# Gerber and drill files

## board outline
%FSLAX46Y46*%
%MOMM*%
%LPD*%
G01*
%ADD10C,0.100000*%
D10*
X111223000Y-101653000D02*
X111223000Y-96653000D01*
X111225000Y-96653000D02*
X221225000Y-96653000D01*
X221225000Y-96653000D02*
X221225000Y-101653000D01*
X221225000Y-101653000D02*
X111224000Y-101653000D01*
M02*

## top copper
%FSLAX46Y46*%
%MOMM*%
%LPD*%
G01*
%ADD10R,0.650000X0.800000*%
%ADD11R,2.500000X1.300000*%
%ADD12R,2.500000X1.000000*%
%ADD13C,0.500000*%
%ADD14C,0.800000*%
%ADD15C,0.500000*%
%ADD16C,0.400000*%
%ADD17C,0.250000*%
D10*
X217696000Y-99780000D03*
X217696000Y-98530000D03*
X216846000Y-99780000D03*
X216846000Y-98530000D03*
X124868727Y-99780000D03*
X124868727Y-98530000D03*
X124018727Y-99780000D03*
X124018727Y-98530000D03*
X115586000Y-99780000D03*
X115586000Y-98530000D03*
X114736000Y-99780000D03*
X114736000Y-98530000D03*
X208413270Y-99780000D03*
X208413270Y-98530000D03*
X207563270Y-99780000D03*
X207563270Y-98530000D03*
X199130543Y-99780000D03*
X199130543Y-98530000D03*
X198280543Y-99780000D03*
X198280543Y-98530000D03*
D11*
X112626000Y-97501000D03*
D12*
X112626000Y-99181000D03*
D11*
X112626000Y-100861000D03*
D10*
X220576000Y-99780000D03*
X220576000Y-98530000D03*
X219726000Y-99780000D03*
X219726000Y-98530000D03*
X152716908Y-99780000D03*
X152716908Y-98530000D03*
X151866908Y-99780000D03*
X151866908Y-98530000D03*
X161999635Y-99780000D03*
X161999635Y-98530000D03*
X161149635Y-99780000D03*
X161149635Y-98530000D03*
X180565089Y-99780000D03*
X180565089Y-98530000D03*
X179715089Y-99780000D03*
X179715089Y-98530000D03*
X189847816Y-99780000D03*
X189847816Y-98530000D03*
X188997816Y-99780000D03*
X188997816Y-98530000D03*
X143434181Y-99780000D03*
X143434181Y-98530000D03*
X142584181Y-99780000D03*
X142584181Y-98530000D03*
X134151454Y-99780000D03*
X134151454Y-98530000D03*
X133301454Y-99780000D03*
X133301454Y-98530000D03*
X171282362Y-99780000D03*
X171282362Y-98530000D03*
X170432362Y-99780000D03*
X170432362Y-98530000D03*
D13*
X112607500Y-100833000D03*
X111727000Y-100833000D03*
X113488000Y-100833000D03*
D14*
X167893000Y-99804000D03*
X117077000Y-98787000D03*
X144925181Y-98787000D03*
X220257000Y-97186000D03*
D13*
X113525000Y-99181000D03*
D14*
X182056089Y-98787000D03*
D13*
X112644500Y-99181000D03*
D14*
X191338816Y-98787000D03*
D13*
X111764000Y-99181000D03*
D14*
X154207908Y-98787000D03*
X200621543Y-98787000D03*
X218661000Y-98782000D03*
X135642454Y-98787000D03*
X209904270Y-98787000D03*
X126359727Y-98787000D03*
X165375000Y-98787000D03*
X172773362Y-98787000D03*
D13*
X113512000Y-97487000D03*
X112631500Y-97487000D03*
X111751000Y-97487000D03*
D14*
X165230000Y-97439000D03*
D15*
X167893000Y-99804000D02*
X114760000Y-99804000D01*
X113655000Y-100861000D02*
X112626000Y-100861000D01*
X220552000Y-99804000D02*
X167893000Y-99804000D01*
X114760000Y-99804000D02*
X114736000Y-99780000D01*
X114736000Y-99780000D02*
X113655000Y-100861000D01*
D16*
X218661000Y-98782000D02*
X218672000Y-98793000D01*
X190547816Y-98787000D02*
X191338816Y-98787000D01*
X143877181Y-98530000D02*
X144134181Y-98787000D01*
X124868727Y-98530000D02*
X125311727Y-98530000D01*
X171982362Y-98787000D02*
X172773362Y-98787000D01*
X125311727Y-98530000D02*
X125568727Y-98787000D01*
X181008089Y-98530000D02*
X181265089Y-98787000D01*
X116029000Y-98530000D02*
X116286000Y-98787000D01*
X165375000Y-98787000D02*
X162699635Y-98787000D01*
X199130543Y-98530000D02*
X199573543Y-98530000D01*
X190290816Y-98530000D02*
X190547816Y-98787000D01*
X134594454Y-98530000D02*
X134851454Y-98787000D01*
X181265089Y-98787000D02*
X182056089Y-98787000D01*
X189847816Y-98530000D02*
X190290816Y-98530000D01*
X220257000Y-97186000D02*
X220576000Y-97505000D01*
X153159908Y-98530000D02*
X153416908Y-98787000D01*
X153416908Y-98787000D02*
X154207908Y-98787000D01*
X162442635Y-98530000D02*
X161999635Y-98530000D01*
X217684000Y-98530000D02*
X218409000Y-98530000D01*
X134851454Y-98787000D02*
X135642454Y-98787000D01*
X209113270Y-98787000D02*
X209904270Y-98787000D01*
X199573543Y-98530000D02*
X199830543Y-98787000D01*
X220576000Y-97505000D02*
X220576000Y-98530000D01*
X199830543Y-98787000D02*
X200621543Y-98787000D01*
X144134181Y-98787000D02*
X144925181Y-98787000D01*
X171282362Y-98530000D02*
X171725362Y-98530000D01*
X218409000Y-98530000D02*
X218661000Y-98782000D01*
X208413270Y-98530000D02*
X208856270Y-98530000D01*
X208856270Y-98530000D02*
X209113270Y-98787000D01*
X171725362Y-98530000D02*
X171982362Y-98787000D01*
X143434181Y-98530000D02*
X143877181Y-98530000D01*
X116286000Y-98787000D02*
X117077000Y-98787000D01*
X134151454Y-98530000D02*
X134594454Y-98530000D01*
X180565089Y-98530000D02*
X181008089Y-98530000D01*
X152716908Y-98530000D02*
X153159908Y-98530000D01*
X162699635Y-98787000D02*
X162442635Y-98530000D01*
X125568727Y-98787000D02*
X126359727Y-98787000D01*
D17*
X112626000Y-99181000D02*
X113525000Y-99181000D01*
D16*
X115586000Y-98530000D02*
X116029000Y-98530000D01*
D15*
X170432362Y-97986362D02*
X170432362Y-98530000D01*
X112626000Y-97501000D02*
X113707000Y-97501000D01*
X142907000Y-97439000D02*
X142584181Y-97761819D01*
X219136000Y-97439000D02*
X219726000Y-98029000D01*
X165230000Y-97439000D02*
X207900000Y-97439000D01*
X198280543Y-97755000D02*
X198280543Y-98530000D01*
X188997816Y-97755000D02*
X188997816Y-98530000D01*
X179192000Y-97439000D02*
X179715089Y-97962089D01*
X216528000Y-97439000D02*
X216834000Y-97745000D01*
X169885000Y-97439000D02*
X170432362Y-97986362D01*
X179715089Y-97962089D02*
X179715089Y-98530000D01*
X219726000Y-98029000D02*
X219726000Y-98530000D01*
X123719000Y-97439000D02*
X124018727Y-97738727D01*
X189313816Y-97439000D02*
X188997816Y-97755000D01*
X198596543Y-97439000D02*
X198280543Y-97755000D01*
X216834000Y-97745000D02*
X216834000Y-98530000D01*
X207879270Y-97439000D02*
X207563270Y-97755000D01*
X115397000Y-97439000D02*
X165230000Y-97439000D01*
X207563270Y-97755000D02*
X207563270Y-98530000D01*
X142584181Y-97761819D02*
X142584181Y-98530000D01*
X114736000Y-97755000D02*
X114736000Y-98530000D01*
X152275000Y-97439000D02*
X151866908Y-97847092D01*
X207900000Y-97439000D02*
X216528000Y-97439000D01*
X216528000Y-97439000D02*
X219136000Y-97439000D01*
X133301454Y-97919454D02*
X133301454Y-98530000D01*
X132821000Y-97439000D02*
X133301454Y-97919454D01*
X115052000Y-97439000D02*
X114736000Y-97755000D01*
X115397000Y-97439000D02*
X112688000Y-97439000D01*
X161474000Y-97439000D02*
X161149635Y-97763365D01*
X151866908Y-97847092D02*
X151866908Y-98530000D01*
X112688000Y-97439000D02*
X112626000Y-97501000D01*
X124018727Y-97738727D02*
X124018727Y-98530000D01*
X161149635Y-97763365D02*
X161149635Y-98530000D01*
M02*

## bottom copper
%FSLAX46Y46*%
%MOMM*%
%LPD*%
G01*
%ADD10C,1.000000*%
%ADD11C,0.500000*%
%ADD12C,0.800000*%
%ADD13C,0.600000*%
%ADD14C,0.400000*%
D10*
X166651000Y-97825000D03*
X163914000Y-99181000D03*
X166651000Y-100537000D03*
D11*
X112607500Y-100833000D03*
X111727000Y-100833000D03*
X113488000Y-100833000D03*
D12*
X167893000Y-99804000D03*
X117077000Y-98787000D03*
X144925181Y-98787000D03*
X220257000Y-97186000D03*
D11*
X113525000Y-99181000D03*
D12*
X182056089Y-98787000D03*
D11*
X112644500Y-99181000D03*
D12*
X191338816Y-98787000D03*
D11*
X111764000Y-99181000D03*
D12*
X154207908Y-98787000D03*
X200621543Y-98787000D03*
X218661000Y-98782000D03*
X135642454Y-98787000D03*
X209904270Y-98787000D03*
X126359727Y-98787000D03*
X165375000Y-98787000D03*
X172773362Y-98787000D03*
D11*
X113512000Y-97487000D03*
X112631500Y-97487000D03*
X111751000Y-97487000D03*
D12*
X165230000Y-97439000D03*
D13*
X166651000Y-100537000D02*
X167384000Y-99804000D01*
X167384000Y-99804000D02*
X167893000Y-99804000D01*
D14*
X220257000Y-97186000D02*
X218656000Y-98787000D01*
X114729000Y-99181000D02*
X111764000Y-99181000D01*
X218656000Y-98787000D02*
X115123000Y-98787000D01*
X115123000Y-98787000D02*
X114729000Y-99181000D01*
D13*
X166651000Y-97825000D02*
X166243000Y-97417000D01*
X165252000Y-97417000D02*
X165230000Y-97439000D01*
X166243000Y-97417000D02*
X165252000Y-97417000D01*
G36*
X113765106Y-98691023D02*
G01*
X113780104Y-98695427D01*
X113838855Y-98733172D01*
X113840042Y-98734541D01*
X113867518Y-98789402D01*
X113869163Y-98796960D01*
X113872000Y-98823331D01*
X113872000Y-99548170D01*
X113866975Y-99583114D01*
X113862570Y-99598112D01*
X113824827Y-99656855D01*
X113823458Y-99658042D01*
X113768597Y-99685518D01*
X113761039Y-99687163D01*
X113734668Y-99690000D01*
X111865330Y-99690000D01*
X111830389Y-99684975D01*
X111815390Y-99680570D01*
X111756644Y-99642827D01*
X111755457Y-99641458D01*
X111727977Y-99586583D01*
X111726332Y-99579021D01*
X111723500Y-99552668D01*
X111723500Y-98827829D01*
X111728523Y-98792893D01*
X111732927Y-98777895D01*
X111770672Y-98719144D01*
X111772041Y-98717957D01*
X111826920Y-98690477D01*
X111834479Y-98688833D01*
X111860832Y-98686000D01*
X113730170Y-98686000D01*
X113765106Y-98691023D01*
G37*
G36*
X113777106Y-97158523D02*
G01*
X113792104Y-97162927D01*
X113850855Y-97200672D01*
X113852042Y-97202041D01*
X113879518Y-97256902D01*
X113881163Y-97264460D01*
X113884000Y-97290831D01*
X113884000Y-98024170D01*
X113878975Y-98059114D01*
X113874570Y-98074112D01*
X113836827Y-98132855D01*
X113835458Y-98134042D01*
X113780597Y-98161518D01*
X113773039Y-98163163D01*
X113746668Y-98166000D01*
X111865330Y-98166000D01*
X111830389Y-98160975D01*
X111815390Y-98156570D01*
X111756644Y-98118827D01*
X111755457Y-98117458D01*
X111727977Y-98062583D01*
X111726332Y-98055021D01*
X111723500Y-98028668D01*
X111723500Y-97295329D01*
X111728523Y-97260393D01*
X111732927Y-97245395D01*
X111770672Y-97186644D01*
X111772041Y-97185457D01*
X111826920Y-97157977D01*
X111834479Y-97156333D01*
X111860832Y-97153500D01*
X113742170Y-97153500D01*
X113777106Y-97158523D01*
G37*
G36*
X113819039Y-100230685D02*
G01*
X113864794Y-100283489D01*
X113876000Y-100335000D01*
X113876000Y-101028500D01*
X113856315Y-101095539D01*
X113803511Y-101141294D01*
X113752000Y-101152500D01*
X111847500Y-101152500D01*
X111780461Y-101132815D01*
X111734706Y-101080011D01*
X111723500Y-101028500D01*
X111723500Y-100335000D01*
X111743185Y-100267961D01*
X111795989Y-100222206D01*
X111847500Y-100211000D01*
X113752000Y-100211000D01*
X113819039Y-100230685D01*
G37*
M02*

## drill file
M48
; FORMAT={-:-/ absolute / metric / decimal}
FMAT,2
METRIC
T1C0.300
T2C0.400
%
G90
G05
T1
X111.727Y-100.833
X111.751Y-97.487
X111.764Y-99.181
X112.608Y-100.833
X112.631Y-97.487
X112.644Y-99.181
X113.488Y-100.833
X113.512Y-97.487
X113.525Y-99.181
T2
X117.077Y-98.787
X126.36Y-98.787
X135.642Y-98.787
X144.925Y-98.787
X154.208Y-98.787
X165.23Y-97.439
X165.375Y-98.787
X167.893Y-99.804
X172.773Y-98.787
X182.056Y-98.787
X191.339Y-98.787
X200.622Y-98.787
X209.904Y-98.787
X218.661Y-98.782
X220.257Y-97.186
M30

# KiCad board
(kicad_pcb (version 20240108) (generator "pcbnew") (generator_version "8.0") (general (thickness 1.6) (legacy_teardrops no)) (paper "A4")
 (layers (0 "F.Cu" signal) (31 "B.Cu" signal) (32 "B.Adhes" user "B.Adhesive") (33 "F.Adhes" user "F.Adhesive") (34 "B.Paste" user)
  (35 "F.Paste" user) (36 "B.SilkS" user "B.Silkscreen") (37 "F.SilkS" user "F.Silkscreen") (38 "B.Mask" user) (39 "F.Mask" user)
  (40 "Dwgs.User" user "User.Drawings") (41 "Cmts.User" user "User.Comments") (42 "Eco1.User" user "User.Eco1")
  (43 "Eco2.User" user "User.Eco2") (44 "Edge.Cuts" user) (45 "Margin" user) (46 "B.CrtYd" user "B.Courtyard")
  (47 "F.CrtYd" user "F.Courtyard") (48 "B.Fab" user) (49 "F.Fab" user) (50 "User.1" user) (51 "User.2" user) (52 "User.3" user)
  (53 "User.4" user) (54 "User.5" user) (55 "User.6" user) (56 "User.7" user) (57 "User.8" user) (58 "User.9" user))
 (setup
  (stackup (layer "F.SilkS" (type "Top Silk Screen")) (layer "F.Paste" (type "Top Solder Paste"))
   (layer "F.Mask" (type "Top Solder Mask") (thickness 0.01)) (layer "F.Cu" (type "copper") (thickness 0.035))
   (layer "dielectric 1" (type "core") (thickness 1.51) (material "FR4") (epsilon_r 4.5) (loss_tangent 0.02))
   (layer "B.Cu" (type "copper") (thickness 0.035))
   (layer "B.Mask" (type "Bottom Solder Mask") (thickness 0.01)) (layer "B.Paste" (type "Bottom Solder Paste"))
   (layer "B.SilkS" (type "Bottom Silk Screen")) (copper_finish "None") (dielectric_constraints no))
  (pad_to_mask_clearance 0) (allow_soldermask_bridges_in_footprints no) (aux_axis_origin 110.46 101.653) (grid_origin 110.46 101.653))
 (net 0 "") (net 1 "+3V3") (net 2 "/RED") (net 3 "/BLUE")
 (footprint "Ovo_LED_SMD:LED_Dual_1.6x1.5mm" (layer "F.Cu") (at 217.271 99.155 90)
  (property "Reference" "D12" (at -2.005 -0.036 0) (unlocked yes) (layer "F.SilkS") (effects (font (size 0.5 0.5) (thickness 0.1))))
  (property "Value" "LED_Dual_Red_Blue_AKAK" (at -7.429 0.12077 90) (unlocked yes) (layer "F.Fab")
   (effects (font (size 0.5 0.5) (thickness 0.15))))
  (pad "1" smd rect (at -0.625 0.425 90) (size 0.8 0.65) (layers "F.Cu" "F.Paste" "F.Mask") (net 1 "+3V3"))
  (pad "2" smd rect (at 0.625 0.425 90) (size 0.8 0.65) (layers "F.Cu" "F.Paste" "F.Mask") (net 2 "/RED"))
  (pad "3" smd rect (at -0.625 -0.425 90) (size 0.8 0.65) (layers "F.Cu" "F.Paste" "F.Mask") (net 1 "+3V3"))
  (pad "4" smd rect (at 0.625 -0.425 90) (size 0.8 0.65) (layers "F.Cu" "F.Paste" "F.Mask") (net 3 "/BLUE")))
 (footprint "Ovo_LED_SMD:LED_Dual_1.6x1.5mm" (layer "F.Cu") (at 124.443727 99.155 90)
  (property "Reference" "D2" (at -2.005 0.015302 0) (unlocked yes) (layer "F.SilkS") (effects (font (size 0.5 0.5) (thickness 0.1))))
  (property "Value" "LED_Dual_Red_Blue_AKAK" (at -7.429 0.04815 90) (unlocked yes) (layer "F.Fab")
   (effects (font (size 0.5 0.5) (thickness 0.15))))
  (pad "1" smd rect (at -0.625 0.425 90) (size 0.8 0.65) (layers "F.Cu" "F.Paste" "F.Mask") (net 1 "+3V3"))
  (pad "2" smd rect (at 0.625 0.425 90) (size 0.8 0.65) (layers "F.Cu" "F.Paste" "F.Mask") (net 2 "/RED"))
  (pad "3" smd rect (at -0.625 -0.425 90) (size 0.8 0.65) (layers "F.Cu" "F.Paste" "F.Mask") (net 1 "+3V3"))
  (pad "4" smd rect (at 0.625 -0.425 90) (size 0.8 0.65) (layers "F.Cu" "F.Paste" "F.Mask") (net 3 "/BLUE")))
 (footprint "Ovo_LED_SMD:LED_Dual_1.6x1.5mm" (layer "F.Cu") (at 115.161 99.155 90)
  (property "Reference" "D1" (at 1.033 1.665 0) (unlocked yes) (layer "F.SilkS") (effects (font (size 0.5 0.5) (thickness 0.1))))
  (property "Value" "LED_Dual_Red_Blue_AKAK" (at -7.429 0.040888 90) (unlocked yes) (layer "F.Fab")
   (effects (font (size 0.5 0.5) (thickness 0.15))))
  (pad "1" smd rect (at -0.625 0.425 90) (size 0.8 0.65) (layers "F.Cu" "F.Paste" "F.Mask") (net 1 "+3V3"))
  (pad "2" smd rect (at 0.625 0.425 90) (size 0.8 0.65) (layers "F.Cu" "F.Paste" "F.Mask") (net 2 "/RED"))
  (pad "3" smd rect (at -0.625 -0.425 90) (size 0.8 0.65) (layers "F.Cu" "F.Paste" "F.Mask") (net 1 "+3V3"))
  (pad "4" smd rect (at 0.625 -0.425 90) (size 0.8 0.65) (layers "F.Cu" "F.Paste" "F.Mask") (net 3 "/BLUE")))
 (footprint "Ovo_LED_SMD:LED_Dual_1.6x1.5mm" (layer "F.Cu") (at 207.98827 99.155 90)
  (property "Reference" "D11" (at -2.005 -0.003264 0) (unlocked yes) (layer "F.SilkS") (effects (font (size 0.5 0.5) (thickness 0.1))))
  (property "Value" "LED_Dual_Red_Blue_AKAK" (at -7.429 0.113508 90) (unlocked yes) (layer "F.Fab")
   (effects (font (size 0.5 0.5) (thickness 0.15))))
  (pad "1" smd rect (at -0.625 0.425 90) (size 0.8 0.65) (layers "F.Cu" "F.Paste" "F.Mask") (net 1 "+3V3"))
  (pad "2" smd rect (at 0.625 0.425 90) (size 0.8 0.65) (layers "F.Cu" "F.Paste" "F.Mask") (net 2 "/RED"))
  (pad "3" smd rect (at -0.625 -0.425 90) (size 0.8 0.65) (layers "F.Cu" "F.Paste" "F.Mask") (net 1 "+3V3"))
  (pad "4" smd rect (at 0.625 -0.425 90) (size 0.8 0.65) (layers "F.Cu" "F.Paste" "F.Mask") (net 3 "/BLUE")))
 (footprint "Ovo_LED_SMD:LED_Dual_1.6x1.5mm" (layer "F.Cu") (at 198.705543 99.155 90)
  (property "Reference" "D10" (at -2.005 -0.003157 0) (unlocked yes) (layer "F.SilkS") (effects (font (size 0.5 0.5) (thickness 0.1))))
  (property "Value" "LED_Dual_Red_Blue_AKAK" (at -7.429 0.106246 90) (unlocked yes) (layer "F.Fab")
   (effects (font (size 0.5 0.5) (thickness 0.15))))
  (pad "1" smd rect (at -0.625 0.425 90) (size 0.8 0.65) (layers "F.Cu" "F.Paste" "F.Mask") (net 1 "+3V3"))
  (pad "2" smd rect (at 0.625 0.425 90) (size 0.8 0.65) (layers "F.Cu" "F.Paste" "F.Mask") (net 2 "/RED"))
  (pad "3" smd rect (at -0.625 -0.425 90) (size 0.8 0.65) (layers "F.Cu" "F.Paste" "F.Mask") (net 1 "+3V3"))
  (pad "4" smd rect (at 0.625 -0.425 90) (size 0.8 0.65) (layers "F.Cu" "F.Paste" "F.Mask") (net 3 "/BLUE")))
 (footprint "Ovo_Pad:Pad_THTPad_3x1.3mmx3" (layer "F.Cu") (at 112.666 97.511)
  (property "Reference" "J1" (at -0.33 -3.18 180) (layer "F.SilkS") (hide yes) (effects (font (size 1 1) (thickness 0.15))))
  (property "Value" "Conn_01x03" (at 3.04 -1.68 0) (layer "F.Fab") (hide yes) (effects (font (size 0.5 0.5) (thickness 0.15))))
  (pad "1" smd rect (at -0.04 -0.01 180) (size 2.5 1.3) (layers "F.Cu" "F.Paste" "F.Mask") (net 3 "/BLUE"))
  (pad "2" smd rect (at -0.04 1.67 180) (size 2.5 1) (layers "F.Cu" "F.Paste" "F.Mask") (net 2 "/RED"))
  (pad "3" smd rect (at -0.04 3.35 180) (size 2.5 1.3) (layers "F.Cu" "F.Paste" "F.Mask") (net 1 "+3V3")))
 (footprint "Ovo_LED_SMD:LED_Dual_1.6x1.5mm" (layer "F.Cu") (at 220.151 99.155 90)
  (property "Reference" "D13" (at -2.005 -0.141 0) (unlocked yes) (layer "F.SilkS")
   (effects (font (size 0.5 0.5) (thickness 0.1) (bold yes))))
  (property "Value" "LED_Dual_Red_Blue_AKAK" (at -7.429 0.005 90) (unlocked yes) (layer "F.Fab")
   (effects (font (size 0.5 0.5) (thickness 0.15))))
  (pad "1" smd rect (at -0.625 0.425 90) (size 0.8 0.65) (layers "F.Cu" "F.Paste" "F.Mask") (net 1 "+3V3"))
  (pad "2" smd rect (at 0.625 0.425 90) (size 0.8 0.65) (layers "F.Cu" "F.Paste" "F.Mask") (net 2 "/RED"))
  (pad "3" smd rect (at -0.625 -0.425 90) (size 0.8 0.65) (layers "F.Cu" "F.Paste" "F.Mask") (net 1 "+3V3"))
  (pad "4" smd rect (at 0.625 -0.425 90) (size 0.8 0.65) (layers "F.Cu" "F.Paste" "F.Mask") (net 3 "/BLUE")))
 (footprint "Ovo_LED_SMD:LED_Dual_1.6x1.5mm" (layer "F.Cu") (at 152.291908 99.155 90)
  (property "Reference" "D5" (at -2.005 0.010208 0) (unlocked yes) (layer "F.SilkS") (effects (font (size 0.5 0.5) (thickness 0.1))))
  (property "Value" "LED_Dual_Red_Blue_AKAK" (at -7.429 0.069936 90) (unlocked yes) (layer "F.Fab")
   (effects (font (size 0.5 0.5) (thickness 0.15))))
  (pad "1" smd rect (at -0.625 0.425 90) (size 0.8 0.65) (layers "F.Cu" "F.Paste" "F.Mask") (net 1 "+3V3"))
  (pad "2" smd rect (at 0.625 0.425 90) (size 0.8 0.65) (layers "F.Cu" "F.Paste" "F.Mask") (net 2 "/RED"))
  (pad "3" smd rect (at -0.625 -0.425 90) (size 0.8 0.65) (layers "F.Cu" "F.Paste" "F.Mask") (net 1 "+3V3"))
  (pad "4" smd rect (at 0.625 -0.425 90) (size 0.8 0.65) (layers "F.Cu" "F.Paste" "F.Mask") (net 3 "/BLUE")))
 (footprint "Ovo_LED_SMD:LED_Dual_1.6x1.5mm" (layer "F.Cu") (at 161.574635 99.155 90)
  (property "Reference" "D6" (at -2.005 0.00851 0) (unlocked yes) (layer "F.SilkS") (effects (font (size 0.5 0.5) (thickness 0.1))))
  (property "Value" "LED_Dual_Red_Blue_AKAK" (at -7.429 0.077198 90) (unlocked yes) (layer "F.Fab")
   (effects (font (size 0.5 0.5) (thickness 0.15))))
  (pad "1" smd rect (at -0.625 0.425 90) (size 0.8 0.65) (layers "F.Cu" "F.Paste" "F.Mask") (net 1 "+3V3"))
  (pad "2" smd rect (at 0.625 0.425 90) (size 0.8 0.65) (layers "F.Cu" "F.Paste" "F.Mask") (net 2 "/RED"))
  (pad "3" smd rect (at -0.625 -0.425 90) (size 0.8 0.65) (layers "F.Cu" "F.Paste" "F.Mask") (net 1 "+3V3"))
  (pad "4" smd rect (at 0.625 -0.425 90) (size 0.8 0.65) (layers "F.Cu" "F.Paste" "F.Mask") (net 3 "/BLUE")))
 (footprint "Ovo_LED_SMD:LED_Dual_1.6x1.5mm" (layer "F.Cu") (at 180.140089 99.155 90)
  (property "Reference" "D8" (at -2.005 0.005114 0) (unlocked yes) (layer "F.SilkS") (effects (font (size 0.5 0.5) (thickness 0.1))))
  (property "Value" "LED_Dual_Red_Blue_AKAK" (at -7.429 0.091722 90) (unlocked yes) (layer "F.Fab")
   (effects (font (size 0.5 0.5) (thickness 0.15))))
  (pad "1" smd rect (at -0.625 0.425 90) (size 0.8 0.65) (layers "F.Cu" "F.Paste" "F.Mask") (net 1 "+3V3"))
  (pad "2" smd rect (at 0.625 0.425 90) (size 0.8 0.65) (layers "F.Cu" "F.Paste" "F.Mask") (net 2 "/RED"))
  (pad "3" smd rect (at -0.625 -0.425 90) (size 0.8 0.65) (layers "F.Cu" "F.Paste" "F.Mask") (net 1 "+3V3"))
  (pad "4" smd rect (at 0.625 -0.425 90) (size 0.8 0.65) (layers "F.Cu" "F.Paste" "F.Mask") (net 3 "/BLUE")))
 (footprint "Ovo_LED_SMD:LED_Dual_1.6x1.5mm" (layer "F.Cu") (at 189.422816 99.155 90)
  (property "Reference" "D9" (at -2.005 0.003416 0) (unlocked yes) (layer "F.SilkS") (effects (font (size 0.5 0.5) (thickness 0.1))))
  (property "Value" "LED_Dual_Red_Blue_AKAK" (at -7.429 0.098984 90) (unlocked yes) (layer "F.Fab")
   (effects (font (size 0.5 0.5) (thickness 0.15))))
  (pad "1" smd rect (at -0.625 0.425 90) (size 0.8 0.65) (layers "F.Cu" "F.Paste" "F.Mask") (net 1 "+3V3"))
  (pad "2" smd rect (at 0.625 0.425 90) (size 0.8 0.65) (layers "F.Cu" "F.Paste" "F.Mask") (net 2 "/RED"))
  (pad "3" smd rect (at -0.625 -0.425 90) (size 0.8 0.65) (layers "F.Cu" "F.Paste" "F.Mask") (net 1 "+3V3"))
  (pad "4" smd rect (at 0.625 -0.425 90) (size 0.8 0.65) (layers "F.Cu" "F.Paste" "F.Mask") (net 3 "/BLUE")))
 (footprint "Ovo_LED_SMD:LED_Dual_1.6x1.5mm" (layer "F.Cu") (at 143.009181 99.155 90)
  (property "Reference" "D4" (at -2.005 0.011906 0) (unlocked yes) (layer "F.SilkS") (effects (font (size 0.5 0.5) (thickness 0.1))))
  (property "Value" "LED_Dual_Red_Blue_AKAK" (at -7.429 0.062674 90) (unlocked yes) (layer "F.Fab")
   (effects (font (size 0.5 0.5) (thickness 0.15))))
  (pad "1" smd rect (at -0.625 0.425 90) (size 0.8 0.65) (layers "F.Cu" "F.Paste" "F.Mask") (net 1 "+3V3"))
  (pad "2" smd rect (at 0.625 0.425 90) (size 0.8 0.65) (layers "F.Cu" "F.Paste" "F.Mask") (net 2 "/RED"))
  (pad "3" smd rect (at -0.625 -0.425 90) (size 0.8 0.65) (layers "F.Cu" "F.Paste" "F.Mask") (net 1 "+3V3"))
  (pad "4" smd rect (at 0.625 -0.425 90) (size 0.8 0.65) (layers "F.Cu" "F.Paste" "F.Mask") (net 3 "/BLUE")))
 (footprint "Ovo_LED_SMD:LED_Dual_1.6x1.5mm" (layer "F.Cu") (at 133.726454 99.155 90)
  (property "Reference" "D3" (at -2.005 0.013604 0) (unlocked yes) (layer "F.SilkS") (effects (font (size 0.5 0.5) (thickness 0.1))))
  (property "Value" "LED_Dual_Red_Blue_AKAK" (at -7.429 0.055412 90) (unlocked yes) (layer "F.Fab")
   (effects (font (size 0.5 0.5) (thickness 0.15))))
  (pad "1" smd rect (at -0.625 0.425 90) (size 0.8 0.65) (layers "F.Cu" "F.Paste" "F.Mask") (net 1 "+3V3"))
  (pad "2" smd rect (at 0.625 0.425 90) (size 0.8 0.65) (layers "F.Cu" "F.Paste" "F.Mask") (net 2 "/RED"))
  (pad "3" smd rect (at -0.625 -0.425 90) (size 0.8 0.65) (layers "F.Cu" "F.Paste" "F.Mask") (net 1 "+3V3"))
  (pad "4" smd rect (at 0.625 -0.425 90) (size 0.8 0.65) (layers "F.Cu" "F.Paste" "F.Mask") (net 3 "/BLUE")))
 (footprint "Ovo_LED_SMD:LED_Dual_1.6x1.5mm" (layer "F.Cu") (at 170.857362 99.155 90)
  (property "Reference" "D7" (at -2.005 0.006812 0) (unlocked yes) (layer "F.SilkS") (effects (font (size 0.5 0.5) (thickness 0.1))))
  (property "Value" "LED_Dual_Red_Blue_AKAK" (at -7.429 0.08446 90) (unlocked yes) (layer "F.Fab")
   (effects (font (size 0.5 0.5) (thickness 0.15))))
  (pad "1" smd rect (at -0.625 0.425 90) (size 0.8 0.65) (layers "F.Cu" "F.Paste" "F.Mask") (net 1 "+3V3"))
  (pad "2" smd rect (at 0.625 0.425 90) (size 0.8 0.65) (layers "F.Cu" "F.Paste" "F.Mask") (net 2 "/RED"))
  (pad "3" smd rect (at -0.625 -0.425 90) (size 0.8 0.65) (layers "F.Cu" "F.Paste" "F.Mask") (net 1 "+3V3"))
  (pad "4" smd rect (at 0.625 -0.425 90) (size 0.8 0.65) (layers "F.Cu" "F.Paste" "F.Mask") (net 3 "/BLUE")))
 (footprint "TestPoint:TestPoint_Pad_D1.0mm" (layer "B.Cu") (at 166.651 97.825 180)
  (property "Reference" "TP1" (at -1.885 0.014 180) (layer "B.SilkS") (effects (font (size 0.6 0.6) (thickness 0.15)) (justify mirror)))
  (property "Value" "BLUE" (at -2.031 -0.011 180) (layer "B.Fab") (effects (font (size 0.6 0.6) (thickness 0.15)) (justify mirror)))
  (pad "1" smd circle (at 0 0 180) (size 1 1) (layers "B.Cu" "B.Mask") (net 3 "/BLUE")))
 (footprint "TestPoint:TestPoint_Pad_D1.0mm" (layer "B.Cu") (at 163.914 99.181 180)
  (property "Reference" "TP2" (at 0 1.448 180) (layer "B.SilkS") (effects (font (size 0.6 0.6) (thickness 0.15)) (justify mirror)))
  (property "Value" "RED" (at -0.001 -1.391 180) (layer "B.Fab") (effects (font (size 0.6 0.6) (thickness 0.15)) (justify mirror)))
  (pad "1" smd circle (at 0 0 180) (size 1 1) (layers "B.Cu" "B.Mask") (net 2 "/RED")))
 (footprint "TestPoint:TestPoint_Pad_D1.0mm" (layer "B.Cu") (at 166.651 100.537 180)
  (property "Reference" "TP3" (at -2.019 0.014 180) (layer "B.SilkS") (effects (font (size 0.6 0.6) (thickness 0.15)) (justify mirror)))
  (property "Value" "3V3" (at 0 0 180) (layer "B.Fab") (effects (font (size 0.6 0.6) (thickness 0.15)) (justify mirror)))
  (pad "1" smd circle (at 0 0 180) (size 1 1) (layers "B.Cu" "B.Mask") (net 1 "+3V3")))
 (gr_line (start 111.223 101.653) (end 111.223 96.653) (stroke (width 0.1) (type default)) (layer "Edge.Cuts"))
 (gr_line (start 111.225 96.653) (end 221.225 96.653) (stroke (width 0.1) (type default)) (layer "Edge.Cuts"))
 (gr_line (start 221.225 96.653) (end 221.225 101.653) (stroke (width 0.1) (type default)) (layer "Edge.Cuts"))
 (gr_line (start 221.225 101.653) (end 111.224 101.653) (stroke (width 0.1) (type default)) (layer "Edge.Cuts"))
 (segment (start 167.893 99.804) (end 114.76 99.804) (width 0.5) (layer "F.Cu") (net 1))
 (segment (start 113.655 100.861) (end 112.626 100.861) (width 0.5) (layer "F.Cu") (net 1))
 (segment (start 220.552 99.804) (end 167.893 99.804) (width 0.5) (layer "F.Cu") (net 1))
 (segment (start 114.76 99.804) (end 114.736 99.78) (width 0.5) (layer "F.Cu") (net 1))
 (segment (start 114.736 99.78) (end 113.655 100.861) (width 0.5) (layer "F.Cu") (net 1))
 (via (at 112.6075 100.833) (size 0.5) (drill 0.3) (layers "F.Cu" "B.Cu") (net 1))
 (via (at 111.727 100.833) (size 0.5) (drill 0.3) (layers "F.Cu" "B.Cu") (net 1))
 (via (at 113.488 100.833) (size 0.5) (drill 0.3) (layers "F.Cu" "B.Cu") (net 1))
 (via (at 167.893 99.804) (size 0.8) (drill 0.4) (layers "F.Cu" "B.Cu") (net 1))
 (segment (start 166.651 100.537) (end 167.384 99.804) (width 0.6) (layer "B.Cu") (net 1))
 (segment (start 167.384 99.804) (end 167.893 99.804) (width 0.6) (layer "B.Cu") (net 1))
 (segment (start 218.661 98.782) (end 218.672 98.793) (width 0.4) (layer "F.Cu") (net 2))
 (segment (start 190.547816 98.787) (end 191.338816 98.787) (width 0.4) (layer "F.Cu") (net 2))
 (segment (start 143.877181 98.53) (end 144.134181 98.787) (width 0.4) (layer "F.Cu") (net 2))
 (segment (start 124.868727 98.53) (end 125.311727 98.53) (width 0.4) (layer "F.Cu") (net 2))
 (segment (start 171.982362 98.787) (end 172.773362 98.787) (width 0.4) (layer "F.Cu") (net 2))
 (segment (start 125.311727 98.53) (end 125.568727 98.787) (width 0.4) (layer "F.Cu") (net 2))
 (segment (start 181.008089 98.53) (end 181.265089 98.787) (width 0.4) (layer "F.Cu") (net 2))
 (segment (start 116.029 98.53) (end 116.286 98.787) (width 0.4) (layer "F.Cu") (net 2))
 (segment (start 165.375 98.787) (end 162.699635 98.787) (width 0.4) (layer "F.Cu") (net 2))
 (segment (start 199.130543 98.53) (end 199.573543 98.53) (width 0.4) (layer "F.Cu") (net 2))
 (segment (start 190.290816 98.53) (end 190.547816 98.787) (width 0.4) (layer "F.Cu") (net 2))
 (segment (start 134.594454 98.53) (end 134.851454 98.787) (width 0.4) (layer "F.Cu") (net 2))
 (segment (start 181.265089 98.787) (end 182.056089 98.787) (width 0.4) (layer "F.Cu") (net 2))
 (segment (start 189.847816 98.53) (end 190.290816 98.53) (width 0.4) (layer "F.Cu") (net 2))
 (segment (start 220.257 97.186) (end 220.576 97.505) (width 0.4) (layer "F.Cu") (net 2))
 (segment (start 153.159908 98.53) (end 153.416908 98.787) (width 0.4) (layer "F.Cu") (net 2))
 (segment (start 153.416908 98.787) (end 154.207908 98.787) (width 0.4) (layer "F.Cu") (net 2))
 (segment (start 162.442635 98.53) (end 161.999635 98.53) (width 0.4) (layer "F.Cu") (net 2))
 (segment (start 217.684 98.53) (end 218.409 98.53) (width 0.4) (layer "F.Cu") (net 2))
 (segment (start 134.851454 98.787) (end 135.642454 98.787) (width 0.4) (layer "F.Cu") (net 2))
 (segment (start 209.11327 98.787) (end 209.90427 98.787) (width 0.4) (layer "F.Cu") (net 2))
 (segment (start 199.573543 98.53) (end 199.830543 98.787) (width 0.4) (layer "F.Cu") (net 2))
 (segment (start 220.576 97.505) (end 220.576 98.53) (width 0.4) (layer "F.Cu") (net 2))
 (segment (start 199.830543 98.787) (end 200.621543 98.787) (width 0.4) (layer "F.Cu") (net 2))
 (segment (start 144.134181 98.787) (end 144.925181 98.787) (width 0.4) (layer "F.Cu") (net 2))
 (segment (start 171.282362 98.53) (end 171.725362 98.53) (width 0.4) (layer "F.Cu") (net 2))
 (segment (start 218.409 98.53) (end 218.661 98.782) (width 0.4) (layer "F.Cu") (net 2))
 (segment (start 208.41327 98.53) (end 208.85627 98.53) (width 0.4) (layer "F.Cu") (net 2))
 (segment (start 208.85627 98.53) (end 209.11327 98.787) (width 0.4) (layer "F.Cu") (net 2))
 (segment (start 171.725362 98.53) (end 171.982362 98.787) (width 0.4) (layer "F.Cu") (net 2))
 (segment (start 143.434181 98.53) (end 143.877181 98.53) (width 0.4) (layer "F.Cu") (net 2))
 (segment (start 116.286 98.787) (end 117.077 98.787) (width 0.4) (layer "F.Cu") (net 2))
 (segment (start 134.151454 98.53) (end 134.594454 98.53) (width 0.4) (layer "F.Cu") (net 2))
 (segment (start 180.565089 98.53) (end 181.008089 98.53) (width 0.4) (layer "F.Cu") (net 2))
 (segment (start 152.716908 98.53) (end 153.159908 98.53) (width 0.4) (layer "F.Cu") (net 2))
 (segment (start 162.699635 98.787) (end 162.442635 98.53) (width 0.4) (layer "F.Cu") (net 2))
 (segment (start 125.568727 98.787) (end 126.359727 98.787) (width 0.4) (layer "F.Cu") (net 2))
 (segment (start 112.626 99.181) (end 113.525 99.181) (width 0.25) (layer "F.Cu") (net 2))
 (segment (start 115.586 98.53) (end 116.029 98.53) (width 0.4) (layer "F.Cu") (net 2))
 (via (at 117.077 98.787) (size 0.8) (drill 0.4) (layers "F.Cu" "B.Cu") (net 2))
 (via (at 144.925181 98.787) (size 0.8) (drill 0.4) (layers "F.Cu" "B.Cu") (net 2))
 (via (at 220.257 97.186) (size 0.8) (drill 0.4) (layers "F.Cu" "B.Cu") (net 2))
 (via (at 113.525 99.181) (size 0.5) (drill 0.3) (layers "F.Cu" "B.Cu") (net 2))
 (via (at 182.056089 98.787) (size 0.8) (drill 0.4) (layers "F.Cu" "B.Cu") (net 2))
 (via (at 112.6445 99.181) (size 0.5) (drill 0.3) (layers "F.Cu" "B.Cu") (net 2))
 (via (at 191.338816 98.787) (size 0.8) (drill 0.4) (layers "F.Cu" "B.Cu") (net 2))
 (via (at 111.764 99.181) (size 0.5) (drill 0.3) (layers "F.Cu" "B.Cu") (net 2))
 (via (at 154.207908 98.787) (size 0.8) (drill 0.4) (layers "F.Cu" "B.Cu") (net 2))
 (via (at 200.621543 98.787) (size 0.8) (drill 0.4) (layers "F.Cu" "B.Cu") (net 2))
 (via (at 218.661 98.782) (size 0.8) (drill 0.4) (layers "F.Cu" "B.Cu") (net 2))
 (via (at 135.642454 98.787) (size 0.8) (drill 0.4) (layers "F.Cu" "B.Cu") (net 2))
 (via (at 209.90427 98.787) (size 0.8) (drill 0.4) (layers "F.Cu" "B.Cu") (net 2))
 (via (at 126.359727 98.787) (size 0.8) (drill 0.4) (layers "F.Cu" "B.Cu") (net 2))
 (via (at 165.375 98.787) (size 0.8) (drill 0.4) (layers "F.Cu" "B.Cu") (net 2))
 (via (at 172.773362 98.787) (size 0.8) (drill 0.4) (layers "F.Cu" "B.Cu") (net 2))
 (segment (start 220.257 97.186) (end 218.656 98.787) (width 0.4) (layer "B.Cu") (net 2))
 (segment (start 114.729 99.181) (end 111.764 99.181) (width 0.4) (layer "B.Cu") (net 2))
 (segment (start 218.656 98.787) (end 115.123 98.787) (width 0.4) (layer "B.Cu") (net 2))
 (segment (start 115.123 98.787) (end 114.729 99.181) (width 0.4) (layer "B.Cu") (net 2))
 (segment (start 170.432362 97.986362) (end 170.432362 98.53) (width 0.5) (layer "F.Cu") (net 3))
 (segment (start 112.626 97.501) (end 113.707 97.501) (width 0.5) (layer "F.Cu") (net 3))
 (segment (start 142.907 97.439) (end 142.584181 97.761819) (width 0.5) (layer "F.Cu") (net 3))
 (segment (start 219.136 97.439) (end 219.726 98.029) (width 0.5) (layer "F.Cu") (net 3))
 (segment (start 165.23 97.439) (end 207.9 97.439) (width 0.5) (layer "F.Cu") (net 3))
 (segment (start 198.280543 97.755) (end 198.280543 98.53) (width 0.5) (layer "F.Cu") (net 3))
 (segment (start 188.997816 97.755) (end 188.997816 98.53) (width 0.5) (layer "F.Cu") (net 3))
 (segment (start 179.192 97.439) (end 179.715089 97.962089) (width 0.5) (layer "F.Cu") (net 3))
 (segment (start 216.528 97.439) (end 216.834 97.745) (width 0.5) (layer "F.Cu") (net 3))
 (segment (start 169.885 97.439) (end 170.432362 97.986362) (width 0.5) (layer "F.Cu") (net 3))
 (segment (start 179.715089 97.962089) (end 179.715089 98.53) (width 0.5) (layer "F.Cu") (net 3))
 (segment (start 219.726 98.029) (end 219.726 98.53) (width 0.5) (layer "F.Cu") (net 3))
 (segment (start 123.719 97.439) (end 124.018727 97.738727) (width 0.5) (layer "F.Cu") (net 3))
 (segment (start 189.313816 97.439) (end 188.997816 97.755) (width 0.5) (layer "F.Cu") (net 3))
 (segment (start 198.596543 97.439) (end 198.280543 97.755) (width 0.5) (layer "F.Cu") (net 3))
 (segment (start 216.834 97.745) (end 216.834 98.53) (width 0.5) (layer "F.Cu") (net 3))
 (segment (start 207.87927 97.439) (end 207.56327 97.755) (width 0.5) (layer "F.Cu") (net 3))
 (segment (start 115.397 97.439) (end 165.23 97.439) (width 0.5) (layer "F.Cu") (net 3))
 (segment (start 207.56327 97.755) (end 207.56327 98.53) (width 0.5) (layer "F.Cu") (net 3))
 (segment (start 142.584181 97.761819) (end 142.584181 98.53) (width 0.5) (layer "F.Cu") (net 3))
 (segment (start 114.736 97.755) (end 114.736 98.53) (width 0.5) (layer "F.Cu") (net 3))
 (segment (start 152.275 97.439) (end 151.866908 97.847092) (width 0.5) (layer "F.Cu") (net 3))
 (segment (start 207.9 97.439) (end 216.528 97.439) (width 0.5) (layer "F.Cu") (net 3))
 (segment (start 216.528 97.439) (end 219.136 97.439) (width 0.5) (layer "F.Cu") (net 3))
 (segment (start 133.301454 97.919454) (end 133.301454 98.53) (width 0.5) (layer "F.Cu") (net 3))
 (segment (start 132.821 97.439) (end 133.301454 97.919454) (width 0.5) (layer "F.Cu") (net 3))
 (segment (start 115.052 97.439) (end 114.736 97.755) (width 0.5) (layer "F.Cu") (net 3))
 (segment (start 115.397 97.439) (end 112.688 97.439) (width 0.5) (layer "F.Cu") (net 3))
 (segment (start 161.474 97.439) (end 161.149635 97.763365) (width 0.5) (layer "F.Cu") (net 3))
 (segment (start 151.866908 97.847092) (end 151.866908 98.53) (width 0.5) (layer "F.Cu") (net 3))
 (segment (start 112.688 97.439) (end 112.626 97.501) (width 0.5) (layer "F.Cu") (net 3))
 (segment (start 124.018727 97.738727) (end 124.018727 98.53) (width 0.5) (layer "F.Cu") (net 3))
 (segment (start 161.149635 97.763365) (end 161.149635 98.53) (width 0.5) (layer "F.Cu") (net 3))
 (via (at 113.512 97.487) (size 0.5) (drill 0.3) (layers "F.Cu" "B.Cu") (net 3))
 (via (at 112.6315 97.487) (size 0.5) (drill 0.3) (layers "F.Cu" "B.Cu") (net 3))
 (via (at 111.751 97.487) (size 0.5) (drill 0.3) (layers "F.Cu" "B.Cu") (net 3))
 (via (at 165.23 97.439) (size 0.8) (drill 0.4) (layers "F.Cu" "B.Cu") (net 3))
 (segment (start 166.651 97.825) (end 166.243 97.417) (width 0.6) (layer "B.Cu") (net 3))
 (segment (start 165.252 97.417) (end 165.23 97.439) (width 0.6) (layer "B.Cu") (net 3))
 (segment (start 166.243 97.417) (end 165.252 97.417) (width 0.6) (layer "B.Cu") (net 3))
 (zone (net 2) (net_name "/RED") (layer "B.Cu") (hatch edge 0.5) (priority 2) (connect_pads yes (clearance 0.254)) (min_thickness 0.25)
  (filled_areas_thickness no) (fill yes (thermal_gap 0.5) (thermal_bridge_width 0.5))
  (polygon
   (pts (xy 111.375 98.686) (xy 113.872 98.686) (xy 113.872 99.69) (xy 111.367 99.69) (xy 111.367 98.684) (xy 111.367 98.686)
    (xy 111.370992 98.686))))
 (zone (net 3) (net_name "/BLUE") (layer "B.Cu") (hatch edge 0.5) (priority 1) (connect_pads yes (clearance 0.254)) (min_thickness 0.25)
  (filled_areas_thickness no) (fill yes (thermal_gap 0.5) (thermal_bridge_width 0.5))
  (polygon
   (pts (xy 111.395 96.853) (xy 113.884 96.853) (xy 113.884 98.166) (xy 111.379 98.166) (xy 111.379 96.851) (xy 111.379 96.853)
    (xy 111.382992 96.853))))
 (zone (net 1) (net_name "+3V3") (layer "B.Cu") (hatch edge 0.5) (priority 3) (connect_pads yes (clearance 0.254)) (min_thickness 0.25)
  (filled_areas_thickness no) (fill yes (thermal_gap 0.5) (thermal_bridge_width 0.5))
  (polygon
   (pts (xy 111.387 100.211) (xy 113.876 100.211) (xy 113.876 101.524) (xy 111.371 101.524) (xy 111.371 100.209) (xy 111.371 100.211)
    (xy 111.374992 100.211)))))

